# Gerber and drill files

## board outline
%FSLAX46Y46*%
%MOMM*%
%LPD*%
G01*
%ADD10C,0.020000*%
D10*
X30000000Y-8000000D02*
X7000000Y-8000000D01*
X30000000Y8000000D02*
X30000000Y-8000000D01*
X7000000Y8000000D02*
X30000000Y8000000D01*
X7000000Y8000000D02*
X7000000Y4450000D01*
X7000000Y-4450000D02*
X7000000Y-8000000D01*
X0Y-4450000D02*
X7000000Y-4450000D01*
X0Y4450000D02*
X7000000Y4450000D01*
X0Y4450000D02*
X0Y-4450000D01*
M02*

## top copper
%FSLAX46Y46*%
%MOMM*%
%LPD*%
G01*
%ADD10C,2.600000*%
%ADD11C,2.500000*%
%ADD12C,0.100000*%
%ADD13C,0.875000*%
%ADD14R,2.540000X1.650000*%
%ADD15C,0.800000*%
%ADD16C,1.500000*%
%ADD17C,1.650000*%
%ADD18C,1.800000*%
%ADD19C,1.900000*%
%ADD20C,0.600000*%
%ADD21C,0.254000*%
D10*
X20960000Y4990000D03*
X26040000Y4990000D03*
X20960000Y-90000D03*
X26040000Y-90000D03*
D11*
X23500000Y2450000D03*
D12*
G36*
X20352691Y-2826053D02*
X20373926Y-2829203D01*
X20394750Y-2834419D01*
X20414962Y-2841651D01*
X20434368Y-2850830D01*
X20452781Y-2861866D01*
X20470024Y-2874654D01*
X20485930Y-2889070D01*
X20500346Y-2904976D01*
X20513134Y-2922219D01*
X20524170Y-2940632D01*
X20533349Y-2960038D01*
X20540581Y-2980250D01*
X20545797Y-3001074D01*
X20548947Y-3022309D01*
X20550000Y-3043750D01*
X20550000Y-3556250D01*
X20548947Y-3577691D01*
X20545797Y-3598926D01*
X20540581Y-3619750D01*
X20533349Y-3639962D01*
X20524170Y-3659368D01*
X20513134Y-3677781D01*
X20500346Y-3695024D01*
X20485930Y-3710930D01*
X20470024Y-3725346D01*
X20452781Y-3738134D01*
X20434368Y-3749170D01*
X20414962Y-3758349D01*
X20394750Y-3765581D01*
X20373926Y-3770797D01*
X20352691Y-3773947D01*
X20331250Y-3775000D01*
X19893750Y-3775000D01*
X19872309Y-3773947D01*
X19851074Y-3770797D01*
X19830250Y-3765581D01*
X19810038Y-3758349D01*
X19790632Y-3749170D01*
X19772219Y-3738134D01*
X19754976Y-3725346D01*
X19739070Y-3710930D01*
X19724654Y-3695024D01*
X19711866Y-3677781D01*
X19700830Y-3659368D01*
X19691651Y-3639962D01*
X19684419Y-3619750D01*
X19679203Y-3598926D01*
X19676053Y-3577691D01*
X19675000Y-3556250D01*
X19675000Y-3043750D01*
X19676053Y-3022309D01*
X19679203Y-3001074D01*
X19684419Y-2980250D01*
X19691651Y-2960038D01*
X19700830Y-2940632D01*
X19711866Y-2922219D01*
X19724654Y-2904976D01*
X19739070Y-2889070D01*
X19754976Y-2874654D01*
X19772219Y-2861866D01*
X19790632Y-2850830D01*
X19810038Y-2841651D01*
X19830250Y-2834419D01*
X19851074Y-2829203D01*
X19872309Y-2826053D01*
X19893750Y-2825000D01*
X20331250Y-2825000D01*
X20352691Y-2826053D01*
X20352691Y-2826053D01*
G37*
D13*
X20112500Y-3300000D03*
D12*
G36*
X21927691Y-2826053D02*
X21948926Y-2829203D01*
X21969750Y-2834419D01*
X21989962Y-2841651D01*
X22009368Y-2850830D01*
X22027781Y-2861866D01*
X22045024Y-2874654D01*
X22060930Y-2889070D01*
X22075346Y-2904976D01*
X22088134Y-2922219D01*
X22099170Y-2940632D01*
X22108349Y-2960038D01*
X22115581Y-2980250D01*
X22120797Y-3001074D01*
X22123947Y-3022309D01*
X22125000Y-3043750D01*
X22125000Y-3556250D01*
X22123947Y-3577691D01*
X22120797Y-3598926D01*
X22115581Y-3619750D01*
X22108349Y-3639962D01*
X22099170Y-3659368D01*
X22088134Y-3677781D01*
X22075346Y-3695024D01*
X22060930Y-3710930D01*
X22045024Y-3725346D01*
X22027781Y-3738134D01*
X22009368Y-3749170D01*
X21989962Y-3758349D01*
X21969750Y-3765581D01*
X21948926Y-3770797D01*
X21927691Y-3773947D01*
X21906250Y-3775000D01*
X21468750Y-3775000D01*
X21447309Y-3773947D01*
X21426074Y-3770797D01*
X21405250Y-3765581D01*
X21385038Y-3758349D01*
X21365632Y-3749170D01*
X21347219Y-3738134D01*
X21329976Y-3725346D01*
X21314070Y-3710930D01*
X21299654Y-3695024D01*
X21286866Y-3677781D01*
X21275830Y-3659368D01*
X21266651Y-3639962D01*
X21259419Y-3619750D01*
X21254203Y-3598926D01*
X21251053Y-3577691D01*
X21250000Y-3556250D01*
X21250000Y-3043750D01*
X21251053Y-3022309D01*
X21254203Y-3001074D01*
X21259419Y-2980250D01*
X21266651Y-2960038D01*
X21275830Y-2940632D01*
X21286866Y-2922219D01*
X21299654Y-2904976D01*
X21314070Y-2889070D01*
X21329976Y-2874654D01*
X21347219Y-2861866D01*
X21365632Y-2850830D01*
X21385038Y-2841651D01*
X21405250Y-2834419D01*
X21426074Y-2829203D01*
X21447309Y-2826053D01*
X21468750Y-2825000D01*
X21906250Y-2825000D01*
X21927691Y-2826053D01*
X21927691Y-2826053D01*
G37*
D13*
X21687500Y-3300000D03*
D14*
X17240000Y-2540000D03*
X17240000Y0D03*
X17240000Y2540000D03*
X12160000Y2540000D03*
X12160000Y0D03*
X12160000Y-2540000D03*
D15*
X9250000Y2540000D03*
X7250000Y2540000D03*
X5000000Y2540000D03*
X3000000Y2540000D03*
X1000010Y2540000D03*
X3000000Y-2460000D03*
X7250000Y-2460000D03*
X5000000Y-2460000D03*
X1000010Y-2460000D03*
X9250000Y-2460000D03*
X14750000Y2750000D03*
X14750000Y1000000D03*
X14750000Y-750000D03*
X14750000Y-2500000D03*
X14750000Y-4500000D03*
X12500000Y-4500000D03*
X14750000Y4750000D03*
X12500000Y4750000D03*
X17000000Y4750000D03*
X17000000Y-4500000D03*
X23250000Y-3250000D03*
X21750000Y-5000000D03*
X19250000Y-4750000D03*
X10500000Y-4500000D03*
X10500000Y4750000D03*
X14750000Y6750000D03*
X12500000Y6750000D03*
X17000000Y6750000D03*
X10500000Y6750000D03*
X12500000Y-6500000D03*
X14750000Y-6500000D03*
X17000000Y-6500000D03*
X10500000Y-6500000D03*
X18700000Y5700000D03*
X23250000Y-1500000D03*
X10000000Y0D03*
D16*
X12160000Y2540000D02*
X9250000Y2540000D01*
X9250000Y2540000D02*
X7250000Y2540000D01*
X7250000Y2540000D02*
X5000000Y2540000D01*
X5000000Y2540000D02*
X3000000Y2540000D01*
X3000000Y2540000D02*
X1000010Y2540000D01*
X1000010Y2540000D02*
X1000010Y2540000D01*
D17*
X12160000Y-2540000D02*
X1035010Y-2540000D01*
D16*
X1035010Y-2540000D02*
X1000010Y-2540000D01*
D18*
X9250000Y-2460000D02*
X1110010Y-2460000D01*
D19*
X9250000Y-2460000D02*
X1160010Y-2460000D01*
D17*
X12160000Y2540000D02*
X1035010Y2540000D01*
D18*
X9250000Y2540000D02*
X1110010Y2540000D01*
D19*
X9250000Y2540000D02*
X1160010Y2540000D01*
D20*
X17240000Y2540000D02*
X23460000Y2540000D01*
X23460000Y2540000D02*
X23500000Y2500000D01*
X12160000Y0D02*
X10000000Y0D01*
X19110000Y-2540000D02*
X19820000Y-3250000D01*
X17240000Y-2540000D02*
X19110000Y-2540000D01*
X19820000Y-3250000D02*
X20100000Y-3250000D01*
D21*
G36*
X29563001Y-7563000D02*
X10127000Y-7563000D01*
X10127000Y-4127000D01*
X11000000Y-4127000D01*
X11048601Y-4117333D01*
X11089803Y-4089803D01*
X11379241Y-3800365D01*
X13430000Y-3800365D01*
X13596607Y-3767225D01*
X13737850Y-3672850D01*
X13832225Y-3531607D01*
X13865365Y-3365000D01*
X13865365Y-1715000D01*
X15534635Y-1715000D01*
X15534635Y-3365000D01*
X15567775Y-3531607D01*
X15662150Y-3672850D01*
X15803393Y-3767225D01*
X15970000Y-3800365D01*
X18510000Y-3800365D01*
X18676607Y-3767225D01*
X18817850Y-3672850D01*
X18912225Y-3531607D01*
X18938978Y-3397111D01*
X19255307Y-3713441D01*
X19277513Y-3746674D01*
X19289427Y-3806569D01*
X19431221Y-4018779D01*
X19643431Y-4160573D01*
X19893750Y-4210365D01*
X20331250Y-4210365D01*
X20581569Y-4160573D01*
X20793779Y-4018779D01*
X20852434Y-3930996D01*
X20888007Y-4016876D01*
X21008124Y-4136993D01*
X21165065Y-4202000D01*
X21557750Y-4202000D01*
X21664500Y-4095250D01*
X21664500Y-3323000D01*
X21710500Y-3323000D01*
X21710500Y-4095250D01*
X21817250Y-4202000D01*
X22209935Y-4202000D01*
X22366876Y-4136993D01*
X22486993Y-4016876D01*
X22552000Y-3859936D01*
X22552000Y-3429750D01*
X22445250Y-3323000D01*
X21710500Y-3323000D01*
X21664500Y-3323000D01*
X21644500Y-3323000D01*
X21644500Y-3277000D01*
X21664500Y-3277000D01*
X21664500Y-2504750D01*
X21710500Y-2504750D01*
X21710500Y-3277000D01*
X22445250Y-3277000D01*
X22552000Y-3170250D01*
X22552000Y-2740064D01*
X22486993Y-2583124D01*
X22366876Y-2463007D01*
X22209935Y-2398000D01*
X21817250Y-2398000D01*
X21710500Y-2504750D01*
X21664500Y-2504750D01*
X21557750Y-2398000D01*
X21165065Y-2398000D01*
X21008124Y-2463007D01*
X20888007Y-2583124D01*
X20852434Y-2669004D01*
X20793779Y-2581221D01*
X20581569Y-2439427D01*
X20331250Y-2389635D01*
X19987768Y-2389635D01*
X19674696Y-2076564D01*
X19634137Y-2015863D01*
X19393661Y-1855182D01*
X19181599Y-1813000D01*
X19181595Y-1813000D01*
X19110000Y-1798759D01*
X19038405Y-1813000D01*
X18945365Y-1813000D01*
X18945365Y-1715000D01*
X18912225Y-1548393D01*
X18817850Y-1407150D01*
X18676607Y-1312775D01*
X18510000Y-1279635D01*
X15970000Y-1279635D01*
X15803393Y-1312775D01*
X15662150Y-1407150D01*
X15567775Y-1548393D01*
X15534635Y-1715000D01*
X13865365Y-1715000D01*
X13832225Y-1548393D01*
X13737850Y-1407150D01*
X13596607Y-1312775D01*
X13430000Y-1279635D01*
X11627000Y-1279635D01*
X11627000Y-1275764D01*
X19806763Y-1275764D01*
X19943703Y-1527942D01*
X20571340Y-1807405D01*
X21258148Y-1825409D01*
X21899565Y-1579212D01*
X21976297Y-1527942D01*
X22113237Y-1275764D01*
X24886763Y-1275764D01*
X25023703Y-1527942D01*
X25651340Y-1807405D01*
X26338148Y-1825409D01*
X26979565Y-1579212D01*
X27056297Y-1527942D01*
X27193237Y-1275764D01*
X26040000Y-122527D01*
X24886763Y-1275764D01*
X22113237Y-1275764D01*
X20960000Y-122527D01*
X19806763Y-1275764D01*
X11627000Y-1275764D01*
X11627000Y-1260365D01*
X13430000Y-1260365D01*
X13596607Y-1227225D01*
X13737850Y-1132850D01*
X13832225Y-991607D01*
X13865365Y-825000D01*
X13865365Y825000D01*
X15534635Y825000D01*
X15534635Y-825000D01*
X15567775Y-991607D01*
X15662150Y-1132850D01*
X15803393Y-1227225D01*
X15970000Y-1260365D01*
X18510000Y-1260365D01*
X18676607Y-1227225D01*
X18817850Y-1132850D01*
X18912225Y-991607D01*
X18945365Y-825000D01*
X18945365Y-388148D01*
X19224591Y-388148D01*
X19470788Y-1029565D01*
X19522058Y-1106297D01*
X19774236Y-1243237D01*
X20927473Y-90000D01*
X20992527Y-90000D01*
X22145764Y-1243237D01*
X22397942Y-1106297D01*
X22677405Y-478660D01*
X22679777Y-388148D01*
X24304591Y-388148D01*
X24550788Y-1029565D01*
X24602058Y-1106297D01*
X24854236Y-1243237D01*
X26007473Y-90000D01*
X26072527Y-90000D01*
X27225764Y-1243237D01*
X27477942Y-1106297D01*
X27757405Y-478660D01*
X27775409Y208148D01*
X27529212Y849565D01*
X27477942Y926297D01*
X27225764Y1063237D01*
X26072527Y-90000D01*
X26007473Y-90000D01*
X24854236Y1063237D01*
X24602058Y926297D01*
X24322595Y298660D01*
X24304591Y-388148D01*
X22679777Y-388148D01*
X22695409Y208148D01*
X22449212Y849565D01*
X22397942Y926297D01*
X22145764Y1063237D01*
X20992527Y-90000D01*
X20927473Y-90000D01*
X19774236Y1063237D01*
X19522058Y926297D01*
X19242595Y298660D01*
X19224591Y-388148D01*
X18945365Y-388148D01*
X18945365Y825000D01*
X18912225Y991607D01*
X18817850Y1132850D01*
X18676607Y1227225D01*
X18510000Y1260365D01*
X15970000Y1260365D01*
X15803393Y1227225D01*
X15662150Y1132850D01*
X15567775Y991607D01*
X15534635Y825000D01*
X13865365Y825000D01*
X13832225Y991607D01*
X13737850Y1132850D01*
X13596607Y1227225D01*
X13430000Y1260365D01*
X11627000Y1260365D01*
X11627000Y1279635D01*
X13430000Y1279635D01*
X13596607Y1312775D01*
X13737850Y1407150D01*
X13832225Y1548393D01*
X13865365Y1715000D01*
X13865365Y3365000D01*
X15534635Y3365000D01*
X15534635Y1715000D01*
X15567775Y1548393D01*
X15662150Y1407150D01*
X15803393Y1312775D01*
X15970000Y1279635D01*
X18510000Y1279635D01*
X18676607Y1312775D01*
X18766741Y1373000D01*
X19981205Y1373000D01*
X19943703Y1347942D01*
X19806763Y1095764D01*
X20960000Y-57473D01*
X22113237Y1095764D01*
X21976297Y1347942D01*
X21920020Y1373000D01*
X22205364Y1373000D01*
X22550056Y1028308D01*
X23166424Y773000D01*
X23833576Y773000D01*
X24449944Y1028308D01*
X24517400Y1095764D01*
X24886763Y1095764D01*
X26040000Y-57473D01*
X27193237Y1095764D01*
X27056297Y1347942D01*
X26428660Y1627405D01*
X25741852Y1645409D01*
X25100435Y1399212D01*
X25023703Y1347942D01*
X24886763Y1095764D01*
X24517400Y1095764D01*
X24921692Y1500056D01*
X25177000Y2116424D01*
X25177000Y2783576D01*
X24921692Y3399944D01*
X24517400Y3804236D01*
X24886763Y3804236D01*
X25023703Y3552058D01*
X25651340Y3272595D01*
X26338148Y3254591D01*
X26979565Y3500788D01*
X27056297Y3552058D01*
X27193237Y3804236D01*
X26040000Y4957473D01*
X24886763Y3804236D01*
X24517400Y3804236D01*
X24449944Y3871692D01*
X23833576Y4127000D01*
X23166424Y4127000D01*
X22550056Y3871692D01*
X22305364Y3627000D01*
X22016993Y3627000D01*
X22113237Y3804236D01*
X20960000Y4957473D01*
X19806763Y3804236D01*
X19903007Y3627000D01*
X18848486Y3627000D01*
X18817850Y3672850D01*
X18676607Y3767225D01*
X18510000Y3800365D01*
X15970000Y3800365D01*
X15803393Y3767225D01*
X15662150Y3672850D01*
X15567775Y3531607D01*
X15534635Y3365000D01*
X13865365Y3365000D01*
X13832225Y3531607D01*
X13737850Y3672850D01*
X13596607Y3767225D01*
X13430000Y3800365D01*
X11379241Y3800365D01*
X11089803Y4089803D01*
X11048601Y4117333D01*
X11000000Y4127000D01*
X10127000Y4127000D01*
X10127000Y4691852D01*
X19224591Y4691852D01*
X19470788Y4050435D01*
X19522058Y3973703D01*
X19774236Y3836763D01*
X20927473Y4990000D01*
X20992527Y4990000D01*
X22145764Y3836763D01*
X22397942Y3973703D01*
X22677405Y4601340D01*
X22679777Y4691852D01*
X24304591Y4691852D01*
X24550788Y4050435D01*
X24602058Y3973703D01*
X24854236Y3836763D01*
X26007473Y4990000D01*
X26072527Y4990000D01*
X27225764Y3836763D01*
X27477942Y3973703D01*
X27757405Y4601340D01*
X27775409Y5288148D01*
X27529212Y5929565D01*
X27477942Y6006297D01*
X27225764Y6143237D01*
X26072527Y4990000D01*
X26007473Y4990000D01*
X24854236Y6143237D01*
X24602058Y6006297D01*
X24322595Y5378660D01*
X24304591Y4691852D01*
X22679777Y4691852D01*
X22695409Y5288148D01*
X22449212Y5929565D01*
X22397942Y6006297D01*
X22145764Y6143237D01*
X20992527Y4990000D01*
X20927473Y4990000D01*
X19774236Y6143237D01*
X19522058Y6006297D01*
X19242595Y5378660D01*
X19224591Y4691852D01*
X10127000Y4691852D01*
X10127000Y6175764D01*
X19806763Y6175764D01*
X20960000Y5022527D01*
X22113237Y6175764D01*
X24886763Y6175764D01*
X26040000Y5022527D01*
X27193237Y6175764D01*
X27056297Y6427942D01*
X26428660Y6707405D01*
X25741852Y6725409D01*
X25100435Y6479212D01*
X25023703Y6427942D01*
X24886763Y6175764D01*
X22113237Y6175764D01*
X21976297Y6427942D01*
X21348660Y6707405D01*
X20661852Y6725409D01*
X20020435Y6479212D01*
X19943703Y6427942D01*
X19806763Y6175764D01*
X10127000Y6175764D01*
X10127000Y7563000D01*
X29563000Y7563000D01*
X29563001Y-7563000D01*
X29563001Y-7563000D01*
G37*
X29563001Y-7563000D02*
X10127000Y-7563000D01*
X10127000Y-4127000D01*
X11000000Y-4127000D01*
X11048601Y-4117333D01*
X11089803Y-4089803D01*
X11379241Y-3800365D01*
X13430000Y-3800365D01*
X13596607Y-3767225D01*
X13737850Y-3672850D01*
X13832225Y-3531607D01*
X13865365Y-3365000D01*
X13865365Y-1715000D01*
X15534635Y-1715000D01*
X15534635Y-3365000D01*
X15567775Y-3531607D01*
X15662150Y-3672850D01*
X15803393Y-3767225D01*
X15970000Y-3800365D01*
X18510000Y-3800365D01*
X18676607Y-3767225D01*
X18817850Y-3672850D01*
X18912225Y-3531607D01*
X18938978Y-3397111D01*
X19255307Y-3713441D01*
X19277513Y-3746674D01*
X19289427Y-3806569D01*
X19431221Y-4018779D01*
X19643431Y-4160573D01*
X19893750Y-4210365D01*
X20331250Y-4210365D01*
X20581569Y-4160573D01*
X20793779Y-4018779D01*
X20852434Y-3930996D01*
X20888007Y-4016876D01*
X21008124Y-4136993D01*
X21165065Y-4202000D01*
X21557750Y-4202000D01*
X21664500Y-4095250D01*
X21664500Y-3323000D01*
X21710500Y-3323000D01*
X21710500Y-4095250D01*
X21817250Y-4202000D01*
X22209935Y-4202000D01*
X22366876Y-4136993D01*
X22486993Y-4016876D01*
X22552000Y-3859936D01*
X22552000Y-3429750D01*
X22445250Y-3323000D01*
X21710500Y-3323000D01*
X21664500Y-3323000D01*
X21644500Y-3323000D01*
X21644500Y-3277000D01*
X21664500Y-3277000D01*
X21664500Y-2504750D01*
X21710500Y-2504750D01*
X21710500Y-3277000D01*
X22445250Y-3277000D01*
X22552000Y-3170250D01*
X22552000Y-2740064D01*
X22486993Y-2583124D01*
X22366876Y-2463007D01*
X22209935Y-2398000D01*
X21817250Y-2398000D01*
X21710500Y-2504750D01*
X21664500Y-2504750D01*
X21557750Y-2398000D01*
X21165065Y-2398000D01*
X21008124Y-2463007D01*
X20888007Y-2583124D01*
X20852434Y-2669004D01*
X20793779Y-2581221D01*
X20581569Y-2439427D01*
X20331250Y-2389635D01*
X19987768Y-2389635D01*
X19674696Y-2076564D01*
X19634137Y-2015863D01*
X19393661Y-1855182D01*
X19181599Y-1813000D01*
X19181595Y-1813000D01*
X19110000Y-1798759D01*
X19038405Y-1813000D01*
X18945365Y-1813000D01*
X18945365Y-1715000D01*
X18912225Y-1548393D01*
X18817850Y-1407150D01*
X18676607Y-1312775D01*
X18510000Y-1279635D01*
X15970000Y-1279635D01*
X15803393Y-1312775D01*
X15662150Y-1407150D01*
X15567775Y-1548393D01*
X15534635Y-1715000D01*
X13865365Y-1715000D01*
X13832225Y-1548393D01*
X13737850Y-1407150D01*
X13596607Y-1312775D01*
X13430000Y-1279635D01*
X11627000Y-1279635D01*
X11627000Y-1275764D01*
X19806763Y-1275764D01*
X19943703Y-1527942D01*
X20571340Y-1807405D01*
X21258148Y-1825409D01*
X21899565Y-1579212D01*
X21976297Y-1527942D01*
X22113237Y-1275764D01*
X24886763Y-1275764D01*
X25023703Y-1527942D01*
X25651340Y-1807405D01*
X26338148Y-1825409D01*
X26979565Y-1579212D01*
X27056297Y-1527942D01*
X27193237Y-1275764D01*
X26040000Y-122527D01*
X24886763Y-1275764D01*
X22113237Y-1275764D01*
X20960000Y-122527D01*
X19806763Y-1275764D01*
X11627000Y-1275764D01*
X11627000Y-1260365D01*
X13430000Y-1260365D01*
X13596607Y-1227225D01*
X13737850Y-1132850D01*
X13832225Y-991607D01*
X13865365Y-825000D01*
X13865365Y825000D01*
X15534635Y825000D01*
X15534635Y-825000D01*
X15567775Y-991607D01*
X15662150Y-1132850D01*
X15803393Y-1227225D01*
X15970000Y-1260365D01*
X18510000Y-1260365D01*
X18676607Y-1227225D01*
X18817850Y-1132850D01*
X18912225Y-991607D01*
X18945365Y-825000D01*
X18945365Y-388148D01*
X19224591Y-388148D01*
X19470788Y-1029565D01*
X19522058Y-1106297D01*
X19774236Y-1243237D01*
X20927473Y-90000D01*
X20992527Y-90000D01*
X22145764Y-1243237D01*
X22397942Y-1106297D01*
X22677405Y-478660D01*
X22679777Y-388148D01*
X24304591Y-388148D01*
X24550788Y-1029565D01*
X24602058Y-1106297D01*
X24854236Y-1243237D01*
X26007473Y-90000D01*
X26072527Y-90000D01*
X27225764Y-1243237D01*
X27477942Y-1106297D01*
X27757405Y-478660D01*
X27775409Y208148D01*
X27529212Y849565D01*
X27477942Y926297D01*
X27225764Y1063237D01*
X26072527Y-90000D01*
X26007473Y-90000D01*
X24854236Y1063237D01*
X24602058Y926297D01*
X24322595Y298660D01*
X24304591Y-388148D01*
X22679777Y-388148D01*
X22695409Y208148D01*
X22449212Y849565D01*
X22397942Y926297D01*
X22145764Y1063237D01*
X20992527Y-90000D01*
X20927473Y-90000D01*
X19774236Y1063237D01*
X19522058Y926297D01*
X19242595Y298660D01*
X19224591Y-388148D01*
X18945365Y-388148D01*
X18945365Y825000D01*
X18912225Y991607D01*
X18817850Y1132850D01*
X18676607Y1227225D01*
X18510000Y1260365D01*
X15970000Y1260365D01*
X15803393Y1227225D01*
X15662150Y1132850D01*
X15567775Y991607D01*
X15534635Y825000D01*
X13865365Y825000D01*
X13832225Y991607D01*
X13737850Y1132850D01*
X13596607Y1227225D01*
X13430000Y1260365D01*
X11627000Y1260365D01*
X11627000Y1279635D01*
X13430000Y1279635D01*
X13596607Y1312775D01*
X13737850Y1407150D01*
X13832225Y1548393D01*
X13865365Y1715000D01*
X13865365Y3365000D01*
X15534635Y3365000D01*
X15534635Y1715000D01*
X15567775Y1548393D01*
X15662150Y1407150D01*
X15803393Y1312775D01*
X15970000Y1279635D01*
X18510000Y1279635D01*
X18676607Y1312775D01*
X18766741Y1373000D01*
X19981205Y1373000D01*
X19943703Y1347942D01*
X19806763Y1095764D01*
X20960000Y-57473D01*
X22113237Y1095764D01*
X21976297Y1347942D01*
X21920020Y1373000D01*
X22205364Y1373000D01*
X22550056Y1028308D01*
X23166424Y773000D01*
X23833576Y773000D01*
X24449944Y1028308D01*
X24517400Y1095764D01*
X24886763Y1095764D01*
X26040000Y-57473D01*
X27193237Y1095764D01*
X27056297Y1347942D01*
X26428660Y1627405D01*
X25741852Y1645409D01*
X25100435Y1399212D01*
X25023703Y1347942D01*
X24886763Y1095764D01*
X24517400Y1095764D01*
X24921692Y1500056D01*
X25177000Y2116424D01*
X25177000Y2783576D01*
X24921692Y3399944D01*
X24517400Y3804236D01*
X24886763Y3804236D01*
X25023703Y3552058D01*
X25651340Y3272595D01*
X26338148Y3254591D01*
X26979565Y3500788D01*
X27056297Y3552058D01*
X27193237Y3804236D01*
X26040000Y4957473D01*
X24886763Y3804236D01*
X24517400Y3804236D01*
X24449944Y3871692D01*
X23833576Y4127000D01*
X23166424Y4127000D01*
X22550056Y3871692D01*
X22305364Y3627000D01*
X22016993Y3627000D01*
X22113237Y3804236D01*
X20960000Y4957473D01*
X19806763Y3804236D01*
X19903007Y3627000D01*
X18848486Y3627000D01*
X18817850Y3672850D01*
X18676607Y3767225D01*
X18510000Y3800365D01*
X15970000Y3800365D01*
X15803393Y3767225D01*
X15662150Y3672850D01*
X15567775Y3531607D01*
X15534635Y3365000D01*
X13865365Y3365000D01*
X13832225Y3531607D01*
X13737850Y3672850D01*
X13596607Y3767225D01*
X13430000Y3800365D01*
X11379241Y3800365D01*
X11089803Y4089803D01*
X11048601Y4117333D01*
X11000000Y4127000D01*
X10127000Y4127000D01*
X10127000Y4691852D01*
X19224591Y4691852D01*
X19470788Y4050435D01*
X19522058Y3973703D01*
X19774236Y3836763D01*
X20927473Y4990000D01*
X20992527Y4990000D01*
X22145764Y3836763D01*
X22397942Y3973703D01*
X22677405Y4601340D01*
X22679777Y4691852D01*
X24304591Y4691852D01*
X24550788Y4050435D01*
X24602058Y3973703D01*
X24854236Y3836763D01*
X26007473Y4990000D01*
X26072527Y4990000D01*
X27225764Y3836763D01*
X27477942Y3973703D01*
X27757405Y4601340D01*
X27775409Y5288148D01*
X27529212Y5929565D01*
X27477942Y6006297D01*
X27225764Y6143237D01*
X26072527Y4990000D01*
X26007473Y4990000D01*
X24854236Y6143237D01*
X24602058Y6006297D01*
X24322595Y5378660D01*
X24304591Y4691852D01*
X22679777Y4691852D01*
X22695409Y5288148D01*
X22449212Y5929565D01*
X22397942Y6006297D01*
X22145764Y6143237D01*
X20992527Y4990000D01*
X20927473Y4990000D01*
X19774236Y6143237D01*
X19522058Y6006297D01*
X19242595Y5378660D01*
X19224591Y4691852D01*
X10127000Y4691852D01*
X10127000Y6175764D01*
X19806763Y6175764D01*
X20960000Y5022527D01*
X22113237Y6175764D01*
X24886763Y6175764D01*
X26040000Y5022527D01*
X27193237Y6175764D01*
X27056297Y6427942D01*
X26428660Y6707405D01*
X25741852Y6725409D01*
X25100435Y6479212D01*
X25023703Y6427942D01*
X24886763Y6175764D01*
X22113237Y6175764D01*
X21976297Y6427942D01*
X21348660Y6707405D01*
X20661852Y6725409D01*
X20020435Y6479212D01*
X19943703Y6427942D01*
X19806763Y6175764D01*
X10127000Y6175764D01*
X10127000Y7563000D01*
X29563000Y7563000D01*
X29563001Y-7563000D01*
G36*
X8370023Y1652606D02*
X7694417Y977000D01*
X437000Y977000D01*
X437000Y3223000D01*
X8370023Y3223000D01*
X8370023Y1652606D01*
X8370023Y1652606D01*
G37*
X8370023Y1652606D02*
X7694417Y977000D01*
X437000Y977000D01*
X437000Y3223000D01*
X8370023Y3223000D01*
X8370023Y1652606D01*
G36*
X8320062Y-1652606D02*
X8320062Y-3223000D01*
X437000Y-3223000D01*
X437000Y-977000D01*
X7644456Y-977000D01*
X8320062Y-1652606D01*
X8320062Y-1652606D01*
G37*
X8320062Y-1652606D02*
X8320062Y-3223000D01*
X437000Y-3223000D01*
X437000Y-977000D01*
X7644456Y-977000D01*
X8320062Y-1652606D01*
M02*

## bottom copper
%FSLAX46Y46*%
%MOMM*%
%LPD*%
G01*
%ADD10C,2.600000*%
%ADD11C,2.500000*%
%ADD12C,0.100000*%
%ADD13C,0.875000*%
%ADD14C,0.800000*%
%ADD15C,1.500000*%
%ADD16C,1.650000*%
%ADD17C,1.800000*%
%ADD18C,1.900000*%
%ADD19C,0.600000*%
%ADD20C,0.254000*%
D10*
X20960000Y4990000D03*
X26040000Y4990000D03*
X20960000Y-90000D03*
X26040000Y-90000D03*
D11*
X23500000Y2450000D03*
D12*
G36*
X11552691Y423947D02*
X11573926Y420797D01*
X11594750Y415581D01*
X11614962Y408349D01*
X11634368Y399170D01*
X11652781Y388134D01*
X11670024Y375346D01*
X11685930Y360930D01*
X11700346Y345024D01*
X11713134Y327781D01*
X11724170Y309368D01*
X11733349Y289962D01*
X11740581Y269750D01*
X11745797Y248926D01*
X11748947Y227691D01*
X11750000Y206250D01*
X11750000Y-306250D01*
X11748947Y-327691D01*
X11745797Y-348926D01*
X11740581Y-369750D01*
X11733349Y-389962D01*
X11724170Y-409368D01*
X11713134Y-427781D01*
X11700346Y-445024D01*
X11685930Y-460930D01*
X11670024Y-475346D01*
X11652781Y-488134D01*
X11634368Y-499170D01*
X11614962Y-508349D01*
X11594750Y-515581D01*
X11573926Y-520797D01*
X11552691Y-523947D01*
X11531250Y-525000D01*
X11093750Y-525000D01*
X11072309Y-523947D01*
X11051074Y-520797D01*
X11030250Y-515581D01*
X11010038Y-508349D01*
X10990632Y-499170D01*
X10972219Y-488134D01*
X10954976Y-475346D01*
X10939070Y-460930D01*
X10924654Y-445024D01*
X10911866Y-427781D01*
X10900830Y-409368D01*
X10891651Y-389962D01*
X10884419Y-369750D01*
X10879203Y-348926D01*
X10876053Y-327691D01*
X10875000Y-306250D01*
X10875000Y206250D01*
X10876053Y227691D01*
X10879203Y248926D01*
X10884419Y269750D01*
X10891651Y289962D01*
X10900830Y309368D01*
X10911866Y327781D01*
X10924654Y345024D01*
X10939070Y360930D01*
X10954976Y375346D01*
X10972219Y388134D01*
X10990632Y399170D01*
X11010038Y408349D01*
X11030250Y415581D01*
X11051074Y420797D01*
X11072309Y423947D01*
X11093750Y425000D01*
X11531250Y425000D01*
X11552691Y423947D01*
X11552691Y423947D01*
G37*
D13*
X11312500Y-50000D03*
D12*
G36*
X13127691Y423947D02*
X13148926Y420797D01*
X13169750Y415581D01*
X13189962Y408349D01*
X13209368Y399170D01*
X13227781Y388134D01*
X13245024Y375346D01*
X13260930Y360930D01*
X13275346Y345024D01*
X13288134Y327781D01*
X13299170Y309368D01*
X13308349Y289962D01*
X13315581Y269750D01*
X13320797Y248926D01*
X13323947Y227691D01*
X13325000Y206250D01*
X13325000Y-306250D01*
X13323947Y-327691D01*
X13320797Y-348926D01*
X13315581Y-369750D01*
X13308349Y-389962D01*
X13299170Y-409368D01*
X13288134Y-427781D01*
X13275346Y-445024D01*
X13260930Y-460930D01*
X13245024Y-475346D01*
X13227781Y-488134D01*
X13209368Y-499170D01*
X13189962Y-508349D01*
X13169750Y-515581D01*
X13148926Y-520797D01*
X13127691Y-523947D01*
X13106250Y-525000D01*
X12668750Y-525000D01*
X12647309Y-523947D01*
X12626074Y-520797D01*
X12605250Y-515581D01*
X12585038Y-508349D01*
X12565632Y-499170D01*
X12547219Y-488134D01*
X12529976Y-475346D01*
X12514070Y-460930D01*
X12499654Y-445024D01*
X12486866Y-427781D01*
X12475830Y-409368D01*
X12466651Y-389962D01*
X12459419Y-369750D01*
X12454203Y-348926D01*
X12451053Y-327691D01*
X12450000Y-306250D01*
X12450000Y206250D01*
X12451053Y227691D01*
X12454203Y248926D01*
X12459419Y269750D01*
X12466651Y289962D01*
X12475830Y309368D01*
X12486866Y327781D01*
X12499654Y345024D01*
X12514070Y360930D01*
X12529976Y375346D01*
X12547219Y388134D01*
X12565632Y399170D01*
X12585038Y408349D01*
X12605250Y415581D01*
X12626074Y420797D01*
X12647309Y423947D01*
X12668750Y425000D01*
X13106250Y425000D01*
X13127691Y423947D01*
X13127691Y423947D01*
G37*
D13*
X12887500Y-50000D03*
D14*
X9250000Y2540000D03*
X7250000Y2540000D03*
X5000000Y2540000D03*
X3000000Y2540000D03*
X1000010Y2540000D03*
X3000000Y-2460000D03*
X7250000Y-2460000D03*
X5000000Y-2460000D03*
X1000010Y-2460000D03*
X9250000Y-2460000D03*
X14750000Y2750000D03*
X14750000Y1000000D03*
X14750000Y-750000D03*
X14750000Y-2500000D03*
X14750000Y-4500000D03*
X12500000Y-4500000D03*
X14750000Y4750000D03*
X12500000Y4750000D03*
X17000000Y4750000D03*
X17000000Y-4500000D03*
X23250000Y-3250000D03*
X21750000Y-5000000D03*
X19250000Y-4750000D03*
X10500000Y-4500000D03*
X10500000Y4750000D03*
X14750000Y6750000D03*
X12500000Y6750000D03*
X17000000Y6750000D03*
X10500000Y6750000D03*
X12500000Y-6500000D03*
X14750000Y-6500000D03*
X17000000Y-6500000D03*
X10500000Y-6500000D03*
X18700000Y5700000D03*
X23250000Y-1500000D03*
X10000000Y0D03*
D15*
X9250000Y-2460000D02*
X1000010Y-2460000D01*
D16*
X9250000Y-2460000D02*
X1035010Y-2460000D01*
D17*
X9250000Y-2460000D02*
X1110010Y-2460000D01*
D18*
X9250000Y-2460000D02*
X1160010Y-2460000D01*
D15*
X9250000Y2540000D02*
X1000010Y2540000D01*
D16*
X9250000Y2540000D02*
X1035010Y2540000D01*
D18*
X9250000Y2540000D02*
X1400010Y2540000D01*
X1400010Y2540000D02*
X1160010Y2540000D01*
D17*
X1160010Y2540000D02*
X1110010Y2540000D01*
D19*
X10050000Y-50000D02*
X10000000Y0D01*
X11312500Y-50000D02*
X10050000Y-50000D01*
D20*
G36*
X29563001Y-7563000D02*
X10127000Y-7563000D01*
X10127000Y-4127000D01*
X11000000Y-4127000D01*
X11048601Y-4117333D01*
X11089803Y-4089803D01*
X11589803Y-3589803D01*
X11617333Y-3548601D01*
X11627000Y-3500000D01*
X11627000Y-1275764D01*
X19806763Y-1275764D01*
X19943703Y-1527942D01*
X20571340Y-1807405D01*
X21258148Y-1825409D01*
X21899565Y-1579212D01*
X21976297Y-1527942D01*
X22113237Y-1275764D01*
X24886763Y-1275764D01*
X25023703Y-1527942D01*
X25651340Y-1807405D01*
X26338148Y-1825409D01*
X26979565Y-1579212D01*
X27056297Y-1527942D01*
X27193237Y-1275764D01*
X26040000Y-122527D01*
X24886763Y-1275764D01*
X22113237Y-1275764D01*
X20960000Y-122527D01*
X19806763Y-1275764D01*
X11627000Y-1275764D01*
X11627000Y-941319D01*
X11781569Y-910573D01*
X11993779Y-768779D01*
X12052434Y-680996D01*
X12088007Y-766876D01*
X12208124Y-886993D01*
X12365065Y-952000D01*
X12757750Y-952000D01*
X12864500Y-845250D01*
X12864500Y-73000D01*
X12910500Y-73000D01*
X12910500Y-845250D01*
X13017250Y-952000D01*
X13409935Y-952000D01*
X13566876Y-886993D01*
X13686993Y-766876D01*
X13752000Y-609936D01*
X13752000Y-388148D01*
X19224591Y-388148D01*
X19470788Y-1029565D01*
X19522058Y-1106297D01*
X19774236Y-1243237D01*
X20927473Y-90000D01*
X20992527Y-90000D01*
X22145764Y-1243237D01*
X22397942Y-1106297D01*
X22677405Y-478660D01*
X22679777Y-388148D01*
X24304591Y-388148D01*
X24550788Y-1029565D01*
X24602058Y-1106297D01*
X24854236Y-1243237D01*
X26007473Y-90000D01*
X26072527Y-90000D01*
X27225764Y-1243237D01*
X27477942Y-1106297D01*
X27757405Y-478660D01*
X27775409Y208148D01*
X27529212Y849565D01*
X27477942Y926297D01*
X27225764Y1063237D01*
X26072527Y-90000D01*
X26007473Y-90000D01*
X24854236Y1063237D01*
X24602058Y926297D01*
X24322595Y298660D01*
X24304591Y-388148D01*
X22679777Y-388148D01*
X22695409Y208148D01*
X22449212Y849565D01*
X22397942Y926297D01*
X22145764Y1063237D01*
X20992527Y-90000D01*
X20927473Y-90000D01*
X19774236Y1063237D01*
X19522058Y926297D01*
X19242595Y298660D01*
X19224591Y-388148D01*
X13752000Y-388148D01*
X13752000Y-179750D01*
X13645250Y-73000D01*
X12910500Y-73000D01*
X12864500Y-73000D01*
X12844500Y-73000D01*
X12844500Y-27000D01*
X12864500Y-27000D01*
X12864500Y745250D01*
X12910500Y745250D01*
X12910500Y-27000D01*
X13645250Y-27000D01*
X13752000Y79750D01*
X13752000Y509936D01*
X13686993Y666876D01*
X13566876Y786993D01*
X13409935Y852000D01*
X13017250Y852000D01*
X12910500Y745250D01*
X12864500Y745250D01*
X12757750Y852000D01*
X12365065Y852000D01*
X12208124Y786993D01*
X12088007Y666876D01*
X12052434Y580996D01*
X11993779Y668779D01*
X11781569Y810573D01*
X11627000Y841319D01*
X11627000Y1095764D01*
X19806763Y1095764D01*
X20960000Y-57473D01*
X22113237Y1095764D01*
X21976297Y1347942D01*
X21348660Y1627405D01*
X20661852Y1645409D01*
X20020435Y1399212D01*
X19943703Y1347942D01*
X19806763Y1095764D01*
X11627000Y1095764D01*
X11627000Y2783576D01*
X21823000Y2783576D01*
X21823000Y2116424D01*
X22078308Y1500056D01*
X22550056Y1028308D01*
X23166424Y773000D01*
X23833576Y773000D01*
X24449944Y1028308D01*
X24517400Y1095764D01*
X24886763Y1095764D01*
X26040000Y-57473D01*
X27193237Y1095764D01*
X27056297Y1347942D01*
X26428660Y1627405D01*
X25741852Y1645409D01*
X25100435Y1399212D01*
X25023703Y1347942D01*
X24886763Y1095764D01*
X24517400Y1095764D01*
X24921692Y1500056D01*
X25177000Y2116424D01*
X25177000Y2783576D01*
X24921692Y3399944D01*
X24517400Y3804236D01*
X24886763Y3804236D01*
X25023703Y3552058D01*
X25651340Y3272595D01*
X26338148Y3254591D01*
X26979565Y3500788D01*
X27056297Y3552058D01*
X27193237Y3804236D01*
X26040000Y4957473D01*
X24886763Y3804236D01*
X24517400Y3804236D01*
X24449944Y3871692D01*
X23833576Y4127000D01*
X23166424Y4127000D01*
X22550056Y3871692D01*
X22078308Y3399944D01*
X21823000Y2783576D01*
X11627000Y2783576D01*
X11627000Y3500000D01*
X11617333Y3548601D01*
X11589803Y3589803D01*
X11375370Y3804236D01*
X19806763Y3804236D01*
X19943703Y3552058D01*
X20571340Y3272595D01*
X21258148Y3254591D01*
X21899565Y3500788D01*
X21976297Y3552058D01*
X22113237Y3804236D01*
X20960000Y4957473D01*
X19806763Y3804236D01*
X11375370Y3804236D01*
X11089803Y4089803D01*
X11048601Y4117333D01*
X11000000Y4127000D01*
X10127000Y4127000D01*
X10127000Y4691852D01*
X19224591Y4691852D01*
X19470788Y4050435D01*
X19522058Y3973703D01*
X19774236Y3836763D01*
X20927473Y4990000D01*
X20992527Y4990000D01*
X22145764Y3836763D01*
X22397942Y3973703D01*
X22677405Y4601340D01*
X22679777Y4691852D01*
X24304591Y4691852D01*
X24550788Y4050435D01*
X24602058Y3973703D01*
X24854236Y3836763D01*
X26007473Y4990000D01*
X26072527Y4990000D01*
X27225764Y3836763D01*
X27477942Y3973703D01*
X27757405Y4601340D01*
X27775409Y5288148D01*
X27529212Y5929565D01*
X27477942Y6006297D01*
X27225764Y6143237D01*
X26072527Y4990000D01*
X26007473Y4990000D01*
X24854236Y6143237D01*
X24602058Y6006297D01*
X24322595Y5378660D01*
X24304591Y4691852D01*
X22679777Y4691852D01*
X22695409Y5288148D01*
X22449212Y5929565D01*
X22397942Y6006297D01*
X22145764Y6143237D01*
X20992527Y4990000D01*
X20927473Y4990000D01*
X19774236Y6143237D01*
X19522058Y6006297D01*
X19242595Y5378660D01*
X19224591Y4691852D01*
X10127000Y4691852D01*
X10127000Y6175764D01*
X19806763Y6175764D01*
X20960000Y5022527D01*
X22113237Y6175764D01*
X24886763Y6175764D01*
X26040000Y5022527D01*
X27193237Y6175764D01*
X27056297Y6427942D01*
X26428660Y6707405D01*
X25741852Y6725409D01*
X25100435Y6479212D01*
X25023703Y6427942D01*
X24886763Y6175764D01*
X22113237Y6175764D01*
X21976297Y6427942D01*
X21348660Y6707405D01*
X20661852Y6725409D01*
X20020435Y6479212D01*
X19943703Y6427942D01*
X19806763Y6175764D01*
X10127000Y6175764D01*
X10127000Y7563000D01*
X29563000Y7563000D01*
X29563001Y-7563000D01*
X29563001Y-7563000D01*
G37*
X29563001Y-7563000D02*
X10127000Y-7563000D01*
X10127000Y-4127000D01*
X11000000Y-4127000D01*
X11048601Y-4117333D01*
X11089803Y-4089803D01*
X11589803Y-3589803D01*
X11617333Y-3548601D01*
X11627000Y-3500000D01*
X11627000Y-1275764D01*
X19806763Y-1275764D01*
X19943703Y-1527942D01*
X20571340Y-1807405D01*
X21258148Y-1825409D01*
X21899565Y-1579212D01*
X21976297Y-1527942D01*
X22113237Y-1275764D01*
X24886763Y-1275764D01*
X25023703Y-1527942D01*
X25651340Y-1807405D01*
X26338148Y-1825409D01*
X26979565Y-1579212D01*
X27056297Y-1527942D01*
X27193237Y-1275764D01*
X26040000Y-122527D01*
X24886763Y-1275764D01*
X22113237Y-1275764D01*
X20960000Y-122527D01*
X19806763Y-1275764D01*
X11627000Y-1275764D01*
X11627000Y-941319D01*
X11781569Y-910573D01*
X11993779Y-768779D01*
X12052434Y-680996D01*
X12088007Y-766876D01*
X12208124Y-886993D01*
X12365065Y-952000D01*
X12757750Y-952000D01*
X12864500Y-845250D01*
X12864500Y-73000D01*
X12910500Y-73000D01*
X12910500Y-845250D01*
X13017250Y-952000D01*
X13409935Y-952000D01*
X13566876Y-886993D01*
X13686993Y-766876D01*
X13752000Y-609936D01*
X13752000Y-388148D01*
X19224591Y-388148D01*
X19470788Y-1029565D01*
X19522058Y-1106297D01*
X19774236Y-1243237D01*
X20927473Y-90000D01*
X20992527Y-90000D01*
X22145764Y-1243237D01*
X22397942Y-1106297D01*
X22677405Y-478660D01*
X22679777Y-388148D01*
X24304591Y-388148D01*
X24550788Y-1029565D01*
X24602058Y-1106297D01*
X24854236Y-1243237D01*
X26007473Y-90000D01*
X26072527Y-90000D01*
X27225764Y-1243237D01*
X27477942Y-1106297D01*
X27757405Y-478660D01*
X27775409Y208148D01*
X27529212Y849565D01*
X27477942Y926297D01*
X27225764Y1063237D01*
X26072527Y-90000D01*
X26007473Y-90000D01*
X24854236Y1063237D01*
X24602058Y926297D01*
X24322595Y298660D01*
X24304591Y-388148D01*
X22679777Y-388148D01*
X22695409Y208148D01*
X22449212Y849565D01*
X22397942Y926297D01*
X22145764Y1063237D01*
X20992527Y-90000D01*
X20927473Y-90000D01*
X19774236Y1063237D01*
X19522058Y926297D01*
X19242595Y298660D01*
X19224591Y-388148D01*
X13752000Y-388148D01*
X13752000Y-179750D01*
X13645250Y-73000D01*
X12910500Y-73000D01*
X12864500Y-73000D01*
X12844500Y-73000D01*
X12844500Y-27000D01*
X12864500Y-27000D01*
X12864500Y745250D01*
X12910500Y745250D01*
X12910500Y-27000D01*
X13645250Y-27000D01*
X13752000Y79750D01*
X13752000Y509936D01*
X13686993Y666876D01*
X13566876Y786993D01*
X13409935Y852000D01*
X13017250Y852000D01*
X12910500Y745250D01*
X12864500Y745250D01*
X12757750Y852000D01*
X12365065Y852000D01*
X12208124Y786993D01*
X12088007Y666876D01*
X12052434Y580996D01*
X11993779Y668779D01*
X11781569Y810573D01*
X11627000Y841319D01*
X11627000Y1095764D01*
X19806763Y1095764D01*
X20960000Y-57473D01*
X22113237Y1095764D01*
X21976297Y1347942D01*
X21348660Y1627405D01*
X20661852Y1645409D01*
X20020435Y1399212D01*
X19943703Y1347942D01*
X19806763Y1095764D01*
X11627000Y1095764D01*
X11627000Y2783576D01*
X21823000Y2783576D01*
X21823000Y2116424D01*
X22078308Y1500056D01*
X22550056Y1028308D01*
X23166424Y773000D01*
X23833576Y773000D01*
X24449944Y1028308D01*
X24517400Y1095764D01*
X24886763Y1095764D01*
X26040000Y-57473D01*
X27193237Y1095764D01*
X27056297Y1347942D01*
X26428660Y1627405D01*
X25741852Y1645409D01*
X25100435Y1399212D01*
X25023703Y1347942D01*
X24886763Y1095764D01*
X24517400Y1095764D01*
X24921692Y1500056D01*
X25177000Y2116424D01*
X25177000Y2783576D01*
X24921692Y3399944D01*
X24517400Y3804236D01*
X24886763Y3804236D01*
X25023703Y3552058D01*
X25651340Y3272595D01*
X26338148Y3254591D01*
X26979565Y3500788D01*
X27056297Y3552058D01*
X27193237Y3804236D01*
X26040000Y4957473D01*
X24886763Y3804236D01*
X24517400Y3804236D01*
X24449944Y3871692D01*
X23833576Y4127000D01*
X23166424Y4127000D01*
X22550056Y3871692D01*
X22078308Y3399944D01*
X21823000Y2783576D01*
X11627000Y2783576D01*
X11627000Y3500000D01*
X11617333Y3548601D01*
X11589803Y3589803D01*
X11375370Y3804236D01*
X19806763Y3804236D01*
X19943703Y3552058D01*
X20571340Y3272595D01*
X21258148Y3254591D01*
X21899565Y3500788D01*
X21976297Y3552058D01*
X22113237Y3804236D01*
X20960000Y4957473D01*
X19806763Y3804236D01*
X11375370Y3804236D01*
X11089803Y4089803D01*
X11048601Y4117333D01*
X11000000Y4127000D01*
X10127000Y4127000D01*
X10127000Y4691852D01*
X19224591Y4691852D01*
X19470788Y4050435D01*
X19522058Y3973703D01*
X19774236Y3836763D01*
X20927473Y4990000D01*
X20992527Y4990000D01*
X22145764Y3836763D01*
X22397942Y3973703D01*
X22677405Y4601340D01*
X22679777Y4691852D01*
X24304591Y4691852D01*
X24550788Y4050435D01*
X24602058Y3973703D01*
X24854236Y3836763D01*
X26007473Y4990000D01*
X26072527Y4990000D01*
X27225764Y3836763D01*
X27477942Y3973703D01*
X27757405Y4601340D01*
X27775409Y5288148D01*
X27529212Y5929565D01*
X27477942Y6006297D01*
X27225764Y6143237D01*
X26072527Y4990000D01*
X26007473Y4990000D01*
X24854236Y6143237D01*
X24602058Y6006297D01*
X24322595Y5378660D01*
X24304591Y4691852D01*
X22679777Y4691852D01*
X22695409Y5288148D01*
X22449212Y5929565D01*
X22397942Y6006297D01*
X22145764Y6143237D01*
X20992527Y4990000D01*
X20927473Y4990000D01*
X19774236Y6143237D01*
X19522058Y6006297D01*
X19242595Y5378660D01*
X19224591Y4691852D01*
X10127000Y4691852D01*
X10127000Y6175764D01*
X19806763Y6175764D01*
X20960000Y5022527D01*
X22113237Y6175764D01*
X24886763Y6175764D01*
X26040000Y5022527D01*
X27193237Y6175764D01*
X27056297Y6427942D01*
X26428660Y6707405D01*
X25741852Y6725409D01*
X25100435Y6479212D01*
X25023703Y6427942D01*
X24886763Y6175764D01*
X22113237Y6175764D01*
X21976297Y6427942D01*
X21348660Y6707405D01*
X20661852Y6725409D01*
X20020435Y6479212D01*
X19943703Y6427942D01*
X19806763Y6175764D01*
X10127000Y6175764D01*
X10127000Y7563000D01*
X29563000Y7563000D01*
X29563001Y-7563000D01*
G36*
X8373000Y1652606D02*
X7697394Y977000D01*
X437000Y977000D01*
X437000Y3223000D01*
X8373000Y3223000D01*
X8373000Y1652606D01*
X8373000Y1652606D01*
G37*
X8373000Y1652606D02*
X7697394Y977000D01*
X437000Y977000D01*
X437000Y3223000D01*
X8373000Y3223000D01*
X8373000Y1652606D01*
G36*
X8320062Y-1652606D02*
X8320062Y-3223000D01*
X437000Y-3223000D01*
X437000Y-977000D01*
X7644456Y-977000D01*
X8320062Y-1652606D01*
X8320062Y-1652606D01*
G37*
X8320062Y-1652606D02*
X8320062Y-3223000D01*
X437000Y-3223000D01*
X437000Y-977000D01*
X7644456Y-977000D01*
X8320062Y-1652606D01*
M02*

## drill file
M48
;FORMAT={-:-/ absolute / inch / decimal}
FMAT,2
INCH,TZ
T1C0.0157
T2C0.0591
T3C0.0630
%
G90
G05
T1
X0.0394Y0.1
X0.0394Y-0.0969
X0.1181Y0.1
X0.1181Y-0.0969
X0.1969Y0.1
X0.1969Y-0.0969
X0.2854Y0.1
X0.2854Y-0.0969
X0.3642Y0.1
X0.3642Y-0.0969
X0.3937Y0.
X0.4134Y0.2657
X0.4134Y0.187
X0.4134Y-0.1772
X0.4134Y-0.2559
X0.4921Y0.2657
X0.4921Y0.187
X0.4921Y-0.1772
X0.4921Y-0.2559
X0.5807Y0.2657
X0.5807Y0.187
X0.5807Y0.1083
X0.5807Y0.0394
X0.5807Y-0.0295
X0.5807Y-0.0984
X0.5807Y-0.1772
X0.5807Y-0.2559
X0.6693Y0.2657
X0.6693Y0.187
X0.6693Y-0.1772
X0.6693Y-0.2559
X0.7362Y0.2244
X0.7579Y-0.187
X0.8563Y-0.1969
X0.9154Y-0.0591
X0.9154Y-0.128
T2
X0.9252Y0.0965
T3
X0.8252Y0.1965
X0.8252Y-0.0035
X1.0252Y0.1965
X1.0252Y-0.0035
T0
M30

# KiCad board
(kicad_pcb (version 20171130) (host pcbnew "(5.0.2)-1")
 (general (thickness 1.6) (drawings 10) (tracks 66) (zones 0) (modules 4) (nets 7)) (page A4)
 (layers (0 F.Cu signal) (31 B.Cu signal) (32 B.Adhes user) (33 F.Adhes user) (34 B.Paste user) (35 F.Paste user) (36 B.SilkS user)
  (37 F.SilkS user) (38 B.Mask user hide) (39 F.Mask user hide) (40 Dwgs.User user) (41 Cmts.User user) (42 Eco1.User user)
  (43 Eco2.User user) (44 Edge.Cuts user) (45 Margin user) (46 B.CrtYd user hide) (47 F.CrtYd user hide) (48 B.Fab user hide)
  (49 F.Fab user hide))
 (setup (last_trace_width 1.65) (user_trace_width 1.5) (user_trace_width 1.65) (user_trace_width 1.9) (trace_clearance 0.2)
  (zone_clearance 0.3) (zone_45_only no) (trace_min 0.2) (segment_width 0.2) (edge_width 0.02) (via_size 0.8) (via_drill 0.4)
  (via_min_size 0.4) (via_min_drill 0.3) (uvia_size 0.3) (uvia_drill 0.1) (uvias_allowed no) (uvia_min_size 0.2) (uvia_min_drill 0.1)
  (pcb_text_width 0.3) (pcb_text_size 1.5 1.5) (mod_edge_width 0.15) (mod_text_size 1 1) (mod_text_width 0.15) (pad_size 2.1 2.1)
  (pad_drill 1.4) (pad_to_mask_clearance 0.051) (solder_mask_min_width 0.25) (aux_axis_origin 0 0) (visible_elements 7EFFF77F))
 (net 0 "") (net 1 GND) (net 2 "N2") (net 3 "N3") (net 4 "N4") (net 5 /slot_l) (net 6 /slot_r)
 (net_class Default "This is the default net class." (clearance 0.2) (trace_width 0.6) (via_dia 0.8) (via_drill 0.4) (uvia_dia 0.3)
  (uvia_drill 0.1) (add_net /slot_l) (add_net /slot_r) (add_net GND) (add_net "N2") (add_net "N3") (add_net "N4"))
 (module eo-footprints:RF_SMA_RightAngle (layer F.Cu) (at 23.5 -2.45 270)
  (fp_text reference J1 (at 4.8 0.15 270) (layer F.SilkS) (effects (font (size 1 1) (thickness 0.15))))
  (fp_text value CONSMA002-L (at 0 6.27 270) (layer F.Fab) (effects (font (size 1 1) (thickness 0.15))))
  (pad 1 thru_hole circle (at -2.54 2.54 270) (size 2.6 2.6) (drill 1.6) (layers *.Cu *.Mask) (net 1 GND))
  (pad 1 thru_hole circle (at -2.54 -2.54 270) (size 2.6 2.6) (drill 1.6) (layers *.Cu *.Mask) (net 1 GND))
  (pad 1 thru_hole circle (at 2.54 2.54 270) (size 2.6 2.6) (drill 1.6) (layers *.Cu *.Mask) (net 1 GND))
  (pad 1 thru_hole circle (at 2.54 -2.54 270) (size 2.6 2.6) (drill 1.6) (layers *.Cu *.Mask) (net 1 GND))
  (pad 2 thru_hole circle (at 0 0 270) (size 2.5 2.5) (drill 1.5) (layers *.Cu *.Mask) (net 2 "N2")))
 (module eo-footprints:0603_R (layer B.Cu) (at 12.1 0.05 180)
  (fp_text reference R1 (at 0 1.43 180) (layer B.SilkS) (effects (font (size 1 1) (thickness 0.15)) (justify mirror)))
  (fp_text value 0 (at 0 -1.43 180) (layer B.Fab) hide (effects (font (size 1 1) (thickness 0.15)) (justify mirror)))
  (pad 2 smd roundrect (at 0.7875 0 180) (size 0.875 0.95) (layers B.Cu B.Paste B.Mask) (roundrect_rratio 0.25) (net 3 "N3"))
  (pad 1 smd roundrect (at -0.7875 0 180) (size 0.875 0.95) (layers B.Cu B.Paste B.Mask) (roundrect_rratio 0.25) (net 1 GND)))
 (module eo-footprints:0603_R (layer F.Cu) (at 20.9 3.3)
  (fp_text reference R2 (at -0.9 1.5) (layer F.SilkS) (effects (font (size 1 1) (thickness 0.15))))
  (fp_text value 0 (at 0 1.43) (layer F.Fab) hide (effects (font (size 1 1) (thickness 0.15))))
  (pad 1 smd roundrect (at -0.7875 0) (size 0.875 0.95) (layers F.Cu F.Paste F.Mask) (roundrect_rratio 0.25) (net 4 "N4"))
  (pad 2 smd roundrect (at 0.7875 0) (size 0.875 0.95) (layers F.Cu F.Paste F.Mask) (roundrect_rratio 0.25) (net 1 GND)))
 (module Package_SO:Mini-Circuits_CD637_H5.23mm (layer F.Cu) (at 14.7 0 180)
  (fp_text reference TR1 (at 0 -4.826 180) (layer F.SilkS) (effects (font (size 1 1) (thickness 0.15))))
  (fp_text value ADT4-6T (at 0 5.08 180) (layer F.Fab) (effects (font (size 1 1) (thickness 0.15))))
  (pad 1 smd rect (at -2.54 -2.54 180) (size 2.54 1.65) (layers F.Cu F.Paste F.Mask) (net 4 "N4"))
  (pad 2 smd rect (at -2.54 0 180) (size 2.54 1.65) (layers F.Cu F.Paste F.Mask))
  (pad 3 smd rect (at -2.54 2.54 180) (size 2.54 1.65) (layers F.Cu F.Paste F.Mask) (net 2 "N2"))
  (pad 4 smd rect (at 2.54 2.54 180) (size 2.54 1.65) (layers F.Cu F.Paste F.Mask) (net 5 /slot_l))
  (pad 5 smd rect (at 2.54 0 180) (size 2.54 1.65) (layers F.Cu F.Paste F.Mask) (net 3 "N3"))
  (pad 6 smd rect (at 2.54 -2.54 180) (size 2.54 1.65) (layers F.Cu F.Paste F.Mask) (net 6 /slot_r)))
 (gr_line (start 30 8) (end 7 8) (layer Edge.Cuts) (width 0.02))
 (gr_line (start 30 -8) (end 30 8) (layer Edge.Cuts) (width 0.02))
 (gr_line (start 7 -8) (end 30 -8) (layer Edge.Cuts) (width 0.02))
 (gr_line (start 7 -8) (end 7 -4.45) (layer Edge.Cuts) (width 0.02))
 (gr_line (start 7 4.45) (end 7 8) (layer Edge.Cuts) (width 0.02))
 (gr_line (start 0 4.45) (end 7 4.45) (layer Edge.Cuts) (width 0.02))
 (gr_line (start 0 -4.45) (end 7 -4.45) (layer Edge.Cuts) (width 0.02))
 (gr_line (start 0 -4.45) (end 0 4.45) (layer Edge.Cuts) (width 0.02))
 (segment (start 12.16 -2.54) (end 9.25 -2.54) (width 1.5) (layer F.Cu) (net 5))
 (segment (start 9.25 -2.54) (end 7.25 -2.54) (width 1.5) (layer F.Cu) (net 5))
 (via (at 9.25 -2.54) (size 0.8) (drill 0.4) (layers F.Cu B.Cu) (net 5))
 (segment (start 7.25 -2.54) (end 5 -2.54) (width 1.5) (layer F.Cu) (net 5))
 (via (at 7.25 -2.54) (size 0.8) (drill 0.4) (layers F.Cu B.Cu) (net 5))
 (segment (start 5 -2.54) (end 3 -2.54) (width 1.5) (layer F.Cu) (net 5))
 (via (at 5 -2.54) (size 0.8) (drill 0.4) (layers F.Cu B.Cu) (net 5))
 (segment (start 3 -2.54) (end 1.00001 -2.54) (width 1.5) (layer F.Cu) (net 5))
 (via (at 3 -2.54) (size 0.8) (drill 0.4) (layers F.Cu B.Cu) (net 5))
 (segment (start 1.00001 -2.54) (end 1.00001 -2.54) (width 1.5) (layer F.Cu) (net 5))
 (via (at 1.00001 -2.54) (size 0.8) (drill 0.4) (layers F.Cu B.Cu) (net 5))
 (via (at 3 2.46) (size 0.8) (drill 0.4) (layers F.Cu B.Cu) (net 6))
 (via (at 7.25 2.46) (size 0.8) (drill 0.4) (layers F.Cu B.Cu) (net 6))
 (via (at 5 2.46) (size 0.8) (drill 0.4) (layers F.Cu B.Cu) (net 6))
 (via (at 1.00001 2.46) (size 0.8) (drill 0.4) (layers F.Cu B.Cu) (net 6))
 (via (at 9.25 2.46) (size 0.8) (drill 0.4) (layers F.Cu B.Cu) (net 6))
 (segment (start 9.25 2.46) (end 1.00001 2.46) (width 1.5) (layer B.Cu) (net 6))
 (segment (start 12.16 2.54) (end 1.03501 2.54) (width 1.65) (layer F.Cu) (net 6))
 (segment (start 1.03501 2.54) (end 1.00001 2.54) (width 1.5) (layer F.Cu) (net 6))
 (segment (start 9.25 2.46) (end 1.03501 2.46) (width 1.65) (layer B.Cu) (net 6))
 (segment (start 9.25 2.46) (end 1.11001 2.46) (width 1.8) (layer F.Cu) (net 6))
 (segment (start 9.25 2.46) (end 1.11001 2.46) (width 1.8) (layer B.Cu) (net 6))
 (segment (start 9.25 2.46) (end 1.16001 2.46) (width 1.9) (layer B.Cu) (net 6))
 (segment (start 9.25 2.46) (end 1.16001 2.46) (width 1.9) (layer F.Cu) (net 6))
 (segment (start 9.25 -2.54) (end 1.00001 -2.54) (width 1.5) (layer B.Cu) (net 5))
 (segment (start 12.16 -2.54) (end 1.03501 -2.54) (width 1.65) (layer F.Cu) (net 5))
 (segment (start 9.25 -2.54) (end 1.03501 -2.54) (width 1.65) (layer B.Cu) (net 5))
 (segment (start 9.25 -2.54) (end 1.11001 -2.54) (width 1.8) (layer F.Cu) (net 5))
 (segment (start 9.25 -2.54) (end 1.40001 -2.54) (width 1.9) (layer B.Cu) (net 5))
 (segment (start 1.40001 -2.54) (end 1.16001 -2.54) (width 1.9) (layer B.Cu) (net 5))
 (segment (start 1.16001 -2.54) (end 1.11001 -2.54) (width 1.8) (layer B.Cu) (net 5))
 (segment (start 9.25 -2.54) (end 1.16001 -2.54) (width 1.9) (layer F.Cu) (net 5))
 (segment (start 17.24 -2.54) (end 23.46 -2.54) (width 0.6) (layer F.Cu) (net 2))
 (segment (start 23.46 -2.54) (end 23.5 -2.5) (width 0.6) (layer F.Cu) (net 2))
 (via (at 14.75 -2.75) (size 0.8) (drill 0.4) (layers F.Cu B.Cu) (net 1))
 (via (at 14.75 -1) (size 0.8) (drill 0.4) (layers F.Cu B.Cu) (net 1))
 (via (at 14.75 0.75) (size 0.8) (drill 0.4) (layers F.Cu B.Cu) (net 1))
 (via (at 14.75 2.5) (size 0.8) (drill 0.4) (layers F.Cu B.Cu) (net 1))
 (via (at 14.75 4.5) (size 0.8) (drill 0.4) (layers F.Cu B.Cu) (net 1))
 (via (at 12.5 4.5) (size 0.8) (drill 0.4) (layers F.Cu B.Cu) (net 1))
 (via (at 14.75 -4.75) (size 0.8) (drill 0.4) (layers F.Cu B.Cu) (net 1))
 (via (at 12.5 -4.75) (size 0.8) (drill 0.4) (layers F.Cu B.Cu) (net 1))
 (via (at 17 -4.75) (size 0.8) (drill 0.4) (layers F.Cu B.Cu) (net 1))
 (via (at 17 4.5) (size 0.8) (drill 0.4) (layers F.Cu B.Cu) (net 1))
 (via (at 23.25 3.25) (size 0.8) (drill 0.4) (layers F.Cu B.Cu) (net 1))
 (via (at 21.75 5) (size 0.8) (drill 0.4) (layers F.Cu B.Cu) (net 1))
 (via (at 19.25 4.75) (size 0.8) (drill 0.4) (layers F.Cu B.Cu) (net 1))
 (via (at 10.5 4.5) (size 0.8) (drill 0.4) (layers F.Cu B.Cu) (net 1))
 (via (at 10.5 -4.75) (size 0.8) (drill 0.4) (layers F.Cu B.Cu) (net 1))
 (via (at 14.75 -6.75) (size 0.8) (drill 0.4) (layers F.Cu B.Cu) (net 1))
 (via (at 12.5 -6.75) (size 0.8) (drill 0.4) (layers F.Cu B.Cu) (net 1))
 (via (at 17 -6.75) (size 0.8) (drill 0.4) (layers F.Cu B.Cu) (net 1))
 (via (at 10.5 -6.75) (size 0.8) (drill 0.4) (layers F.Cu B.Cu) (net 1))
 (via (at 12.5 6.5) (size 0.8) (drill 0.4) (layers F.Cu B.Cu) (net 1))
 (via (at 14.75 6.5) (size 0.8) (drill 0.4) (layers F.Cu B.Cu) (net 1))
 (via (at 17 6.5) (size 0.8) (drill 0.4) (layers F.Cu B.Cu) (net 1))
 (via (at 10.5 6.5) (size 0.8) (drill 0.4) (layers F.Cu B.Cu) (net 1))
 (via (at 18.7 -5.7) (size 0.8) (drill 0.4) (layers F.Cu B.Cu) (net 1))
 (via (at 23.25 1.5) (size 0.8) (drill 0.4) (layers F.Cu B.Cu) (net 1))
 (via (at 10 0) (size 0.8) (drill 0.4) (layers F.Cu B.Cu) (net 3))
 (segment (start 12.16 0) (end 10 0) (width 0.6) (layer F.Cu) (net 3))
 (segment (start 10.05 0.05) (end 10 0) (width 0.6) (layer B.Cu) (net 3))
 (segment (start 11.3125 0.05) (end 10.05 0.05) (width 0.6) (layer B.Cu) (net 3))
 (segment (start 19.11 2.54) (end 19.82 3.25) (width 0.6) (layer F.Cu) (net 4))
 (segment (start 17.24 2.54) (end 19.11 2.54) (width 0.6) (layer F.Cu) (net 4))
 (segment (start 19.82 3.25) (end 20.1 3.25) (width 0.6) (layer F.Cu) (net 4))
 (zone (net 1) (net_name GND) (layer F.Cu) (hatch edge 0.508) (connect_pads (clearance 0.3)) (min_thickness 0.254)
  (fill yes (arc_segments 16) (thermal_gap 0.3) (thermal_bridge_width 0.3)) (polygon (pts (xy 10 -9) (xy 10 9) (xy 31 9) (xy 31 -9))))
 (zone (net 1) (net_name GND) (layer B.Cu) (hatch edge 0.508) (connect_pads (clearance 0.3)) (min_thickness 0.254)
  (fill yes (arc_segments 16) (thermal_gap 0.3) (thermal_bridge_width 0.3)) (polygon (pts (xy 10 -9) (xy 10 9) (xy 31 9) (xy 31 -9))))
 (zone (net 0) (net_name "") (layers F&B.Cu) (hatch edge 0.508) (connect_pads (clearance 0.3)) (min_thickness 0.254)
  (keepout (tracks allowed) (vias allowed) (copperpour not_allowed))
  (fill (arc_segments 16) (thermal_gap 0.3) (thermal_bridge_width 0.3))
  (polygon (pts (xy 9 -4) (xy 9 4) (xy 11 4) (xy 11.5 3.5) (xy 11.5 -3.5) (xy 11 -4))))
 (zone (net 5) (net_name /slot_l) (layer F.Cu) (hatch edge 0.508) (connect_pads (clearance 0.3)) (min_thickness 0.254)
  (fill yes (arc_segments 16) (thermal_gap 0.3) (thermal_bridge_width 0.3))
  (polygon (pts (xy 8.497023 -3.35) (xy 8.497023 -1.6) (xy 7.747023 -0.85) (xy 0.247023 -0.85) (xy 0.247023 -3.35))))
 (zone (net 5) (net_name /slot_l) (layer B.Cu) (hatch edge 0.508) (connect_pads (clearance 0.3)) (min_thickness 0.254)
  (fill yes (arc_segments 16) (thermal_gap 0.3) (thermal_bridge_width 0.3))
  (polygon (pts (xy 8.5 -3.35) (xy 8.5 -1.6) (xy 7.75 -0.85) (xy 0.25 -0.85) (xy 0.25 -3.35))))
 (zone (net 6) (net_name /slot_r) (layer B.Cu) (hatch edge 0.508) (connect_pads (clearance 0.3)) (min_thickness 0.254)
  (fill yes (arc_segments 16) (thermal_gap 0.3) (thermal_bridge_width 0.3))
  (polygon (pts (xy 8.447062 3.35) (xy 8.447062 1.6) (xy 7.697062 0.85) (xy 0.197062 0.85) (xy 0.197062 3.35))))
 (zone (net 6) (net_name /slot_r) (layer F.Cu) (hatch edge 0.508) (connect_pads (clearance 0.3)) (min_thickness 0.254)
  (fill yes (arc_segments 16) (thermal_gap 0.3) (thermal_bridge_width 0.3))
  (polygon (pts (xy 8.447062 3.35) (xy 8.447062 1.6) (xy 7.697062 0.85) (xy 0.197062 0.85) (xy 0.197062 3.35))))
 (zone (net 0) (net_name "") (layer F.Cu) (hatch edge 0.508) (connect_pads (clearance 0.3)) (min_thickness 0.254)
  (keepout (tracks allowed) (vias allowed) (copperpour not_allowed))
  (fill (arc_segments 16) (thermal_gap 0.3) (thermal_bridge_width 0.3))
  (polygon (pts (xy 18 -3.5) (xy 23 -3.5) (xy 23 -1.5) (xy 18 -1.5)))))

